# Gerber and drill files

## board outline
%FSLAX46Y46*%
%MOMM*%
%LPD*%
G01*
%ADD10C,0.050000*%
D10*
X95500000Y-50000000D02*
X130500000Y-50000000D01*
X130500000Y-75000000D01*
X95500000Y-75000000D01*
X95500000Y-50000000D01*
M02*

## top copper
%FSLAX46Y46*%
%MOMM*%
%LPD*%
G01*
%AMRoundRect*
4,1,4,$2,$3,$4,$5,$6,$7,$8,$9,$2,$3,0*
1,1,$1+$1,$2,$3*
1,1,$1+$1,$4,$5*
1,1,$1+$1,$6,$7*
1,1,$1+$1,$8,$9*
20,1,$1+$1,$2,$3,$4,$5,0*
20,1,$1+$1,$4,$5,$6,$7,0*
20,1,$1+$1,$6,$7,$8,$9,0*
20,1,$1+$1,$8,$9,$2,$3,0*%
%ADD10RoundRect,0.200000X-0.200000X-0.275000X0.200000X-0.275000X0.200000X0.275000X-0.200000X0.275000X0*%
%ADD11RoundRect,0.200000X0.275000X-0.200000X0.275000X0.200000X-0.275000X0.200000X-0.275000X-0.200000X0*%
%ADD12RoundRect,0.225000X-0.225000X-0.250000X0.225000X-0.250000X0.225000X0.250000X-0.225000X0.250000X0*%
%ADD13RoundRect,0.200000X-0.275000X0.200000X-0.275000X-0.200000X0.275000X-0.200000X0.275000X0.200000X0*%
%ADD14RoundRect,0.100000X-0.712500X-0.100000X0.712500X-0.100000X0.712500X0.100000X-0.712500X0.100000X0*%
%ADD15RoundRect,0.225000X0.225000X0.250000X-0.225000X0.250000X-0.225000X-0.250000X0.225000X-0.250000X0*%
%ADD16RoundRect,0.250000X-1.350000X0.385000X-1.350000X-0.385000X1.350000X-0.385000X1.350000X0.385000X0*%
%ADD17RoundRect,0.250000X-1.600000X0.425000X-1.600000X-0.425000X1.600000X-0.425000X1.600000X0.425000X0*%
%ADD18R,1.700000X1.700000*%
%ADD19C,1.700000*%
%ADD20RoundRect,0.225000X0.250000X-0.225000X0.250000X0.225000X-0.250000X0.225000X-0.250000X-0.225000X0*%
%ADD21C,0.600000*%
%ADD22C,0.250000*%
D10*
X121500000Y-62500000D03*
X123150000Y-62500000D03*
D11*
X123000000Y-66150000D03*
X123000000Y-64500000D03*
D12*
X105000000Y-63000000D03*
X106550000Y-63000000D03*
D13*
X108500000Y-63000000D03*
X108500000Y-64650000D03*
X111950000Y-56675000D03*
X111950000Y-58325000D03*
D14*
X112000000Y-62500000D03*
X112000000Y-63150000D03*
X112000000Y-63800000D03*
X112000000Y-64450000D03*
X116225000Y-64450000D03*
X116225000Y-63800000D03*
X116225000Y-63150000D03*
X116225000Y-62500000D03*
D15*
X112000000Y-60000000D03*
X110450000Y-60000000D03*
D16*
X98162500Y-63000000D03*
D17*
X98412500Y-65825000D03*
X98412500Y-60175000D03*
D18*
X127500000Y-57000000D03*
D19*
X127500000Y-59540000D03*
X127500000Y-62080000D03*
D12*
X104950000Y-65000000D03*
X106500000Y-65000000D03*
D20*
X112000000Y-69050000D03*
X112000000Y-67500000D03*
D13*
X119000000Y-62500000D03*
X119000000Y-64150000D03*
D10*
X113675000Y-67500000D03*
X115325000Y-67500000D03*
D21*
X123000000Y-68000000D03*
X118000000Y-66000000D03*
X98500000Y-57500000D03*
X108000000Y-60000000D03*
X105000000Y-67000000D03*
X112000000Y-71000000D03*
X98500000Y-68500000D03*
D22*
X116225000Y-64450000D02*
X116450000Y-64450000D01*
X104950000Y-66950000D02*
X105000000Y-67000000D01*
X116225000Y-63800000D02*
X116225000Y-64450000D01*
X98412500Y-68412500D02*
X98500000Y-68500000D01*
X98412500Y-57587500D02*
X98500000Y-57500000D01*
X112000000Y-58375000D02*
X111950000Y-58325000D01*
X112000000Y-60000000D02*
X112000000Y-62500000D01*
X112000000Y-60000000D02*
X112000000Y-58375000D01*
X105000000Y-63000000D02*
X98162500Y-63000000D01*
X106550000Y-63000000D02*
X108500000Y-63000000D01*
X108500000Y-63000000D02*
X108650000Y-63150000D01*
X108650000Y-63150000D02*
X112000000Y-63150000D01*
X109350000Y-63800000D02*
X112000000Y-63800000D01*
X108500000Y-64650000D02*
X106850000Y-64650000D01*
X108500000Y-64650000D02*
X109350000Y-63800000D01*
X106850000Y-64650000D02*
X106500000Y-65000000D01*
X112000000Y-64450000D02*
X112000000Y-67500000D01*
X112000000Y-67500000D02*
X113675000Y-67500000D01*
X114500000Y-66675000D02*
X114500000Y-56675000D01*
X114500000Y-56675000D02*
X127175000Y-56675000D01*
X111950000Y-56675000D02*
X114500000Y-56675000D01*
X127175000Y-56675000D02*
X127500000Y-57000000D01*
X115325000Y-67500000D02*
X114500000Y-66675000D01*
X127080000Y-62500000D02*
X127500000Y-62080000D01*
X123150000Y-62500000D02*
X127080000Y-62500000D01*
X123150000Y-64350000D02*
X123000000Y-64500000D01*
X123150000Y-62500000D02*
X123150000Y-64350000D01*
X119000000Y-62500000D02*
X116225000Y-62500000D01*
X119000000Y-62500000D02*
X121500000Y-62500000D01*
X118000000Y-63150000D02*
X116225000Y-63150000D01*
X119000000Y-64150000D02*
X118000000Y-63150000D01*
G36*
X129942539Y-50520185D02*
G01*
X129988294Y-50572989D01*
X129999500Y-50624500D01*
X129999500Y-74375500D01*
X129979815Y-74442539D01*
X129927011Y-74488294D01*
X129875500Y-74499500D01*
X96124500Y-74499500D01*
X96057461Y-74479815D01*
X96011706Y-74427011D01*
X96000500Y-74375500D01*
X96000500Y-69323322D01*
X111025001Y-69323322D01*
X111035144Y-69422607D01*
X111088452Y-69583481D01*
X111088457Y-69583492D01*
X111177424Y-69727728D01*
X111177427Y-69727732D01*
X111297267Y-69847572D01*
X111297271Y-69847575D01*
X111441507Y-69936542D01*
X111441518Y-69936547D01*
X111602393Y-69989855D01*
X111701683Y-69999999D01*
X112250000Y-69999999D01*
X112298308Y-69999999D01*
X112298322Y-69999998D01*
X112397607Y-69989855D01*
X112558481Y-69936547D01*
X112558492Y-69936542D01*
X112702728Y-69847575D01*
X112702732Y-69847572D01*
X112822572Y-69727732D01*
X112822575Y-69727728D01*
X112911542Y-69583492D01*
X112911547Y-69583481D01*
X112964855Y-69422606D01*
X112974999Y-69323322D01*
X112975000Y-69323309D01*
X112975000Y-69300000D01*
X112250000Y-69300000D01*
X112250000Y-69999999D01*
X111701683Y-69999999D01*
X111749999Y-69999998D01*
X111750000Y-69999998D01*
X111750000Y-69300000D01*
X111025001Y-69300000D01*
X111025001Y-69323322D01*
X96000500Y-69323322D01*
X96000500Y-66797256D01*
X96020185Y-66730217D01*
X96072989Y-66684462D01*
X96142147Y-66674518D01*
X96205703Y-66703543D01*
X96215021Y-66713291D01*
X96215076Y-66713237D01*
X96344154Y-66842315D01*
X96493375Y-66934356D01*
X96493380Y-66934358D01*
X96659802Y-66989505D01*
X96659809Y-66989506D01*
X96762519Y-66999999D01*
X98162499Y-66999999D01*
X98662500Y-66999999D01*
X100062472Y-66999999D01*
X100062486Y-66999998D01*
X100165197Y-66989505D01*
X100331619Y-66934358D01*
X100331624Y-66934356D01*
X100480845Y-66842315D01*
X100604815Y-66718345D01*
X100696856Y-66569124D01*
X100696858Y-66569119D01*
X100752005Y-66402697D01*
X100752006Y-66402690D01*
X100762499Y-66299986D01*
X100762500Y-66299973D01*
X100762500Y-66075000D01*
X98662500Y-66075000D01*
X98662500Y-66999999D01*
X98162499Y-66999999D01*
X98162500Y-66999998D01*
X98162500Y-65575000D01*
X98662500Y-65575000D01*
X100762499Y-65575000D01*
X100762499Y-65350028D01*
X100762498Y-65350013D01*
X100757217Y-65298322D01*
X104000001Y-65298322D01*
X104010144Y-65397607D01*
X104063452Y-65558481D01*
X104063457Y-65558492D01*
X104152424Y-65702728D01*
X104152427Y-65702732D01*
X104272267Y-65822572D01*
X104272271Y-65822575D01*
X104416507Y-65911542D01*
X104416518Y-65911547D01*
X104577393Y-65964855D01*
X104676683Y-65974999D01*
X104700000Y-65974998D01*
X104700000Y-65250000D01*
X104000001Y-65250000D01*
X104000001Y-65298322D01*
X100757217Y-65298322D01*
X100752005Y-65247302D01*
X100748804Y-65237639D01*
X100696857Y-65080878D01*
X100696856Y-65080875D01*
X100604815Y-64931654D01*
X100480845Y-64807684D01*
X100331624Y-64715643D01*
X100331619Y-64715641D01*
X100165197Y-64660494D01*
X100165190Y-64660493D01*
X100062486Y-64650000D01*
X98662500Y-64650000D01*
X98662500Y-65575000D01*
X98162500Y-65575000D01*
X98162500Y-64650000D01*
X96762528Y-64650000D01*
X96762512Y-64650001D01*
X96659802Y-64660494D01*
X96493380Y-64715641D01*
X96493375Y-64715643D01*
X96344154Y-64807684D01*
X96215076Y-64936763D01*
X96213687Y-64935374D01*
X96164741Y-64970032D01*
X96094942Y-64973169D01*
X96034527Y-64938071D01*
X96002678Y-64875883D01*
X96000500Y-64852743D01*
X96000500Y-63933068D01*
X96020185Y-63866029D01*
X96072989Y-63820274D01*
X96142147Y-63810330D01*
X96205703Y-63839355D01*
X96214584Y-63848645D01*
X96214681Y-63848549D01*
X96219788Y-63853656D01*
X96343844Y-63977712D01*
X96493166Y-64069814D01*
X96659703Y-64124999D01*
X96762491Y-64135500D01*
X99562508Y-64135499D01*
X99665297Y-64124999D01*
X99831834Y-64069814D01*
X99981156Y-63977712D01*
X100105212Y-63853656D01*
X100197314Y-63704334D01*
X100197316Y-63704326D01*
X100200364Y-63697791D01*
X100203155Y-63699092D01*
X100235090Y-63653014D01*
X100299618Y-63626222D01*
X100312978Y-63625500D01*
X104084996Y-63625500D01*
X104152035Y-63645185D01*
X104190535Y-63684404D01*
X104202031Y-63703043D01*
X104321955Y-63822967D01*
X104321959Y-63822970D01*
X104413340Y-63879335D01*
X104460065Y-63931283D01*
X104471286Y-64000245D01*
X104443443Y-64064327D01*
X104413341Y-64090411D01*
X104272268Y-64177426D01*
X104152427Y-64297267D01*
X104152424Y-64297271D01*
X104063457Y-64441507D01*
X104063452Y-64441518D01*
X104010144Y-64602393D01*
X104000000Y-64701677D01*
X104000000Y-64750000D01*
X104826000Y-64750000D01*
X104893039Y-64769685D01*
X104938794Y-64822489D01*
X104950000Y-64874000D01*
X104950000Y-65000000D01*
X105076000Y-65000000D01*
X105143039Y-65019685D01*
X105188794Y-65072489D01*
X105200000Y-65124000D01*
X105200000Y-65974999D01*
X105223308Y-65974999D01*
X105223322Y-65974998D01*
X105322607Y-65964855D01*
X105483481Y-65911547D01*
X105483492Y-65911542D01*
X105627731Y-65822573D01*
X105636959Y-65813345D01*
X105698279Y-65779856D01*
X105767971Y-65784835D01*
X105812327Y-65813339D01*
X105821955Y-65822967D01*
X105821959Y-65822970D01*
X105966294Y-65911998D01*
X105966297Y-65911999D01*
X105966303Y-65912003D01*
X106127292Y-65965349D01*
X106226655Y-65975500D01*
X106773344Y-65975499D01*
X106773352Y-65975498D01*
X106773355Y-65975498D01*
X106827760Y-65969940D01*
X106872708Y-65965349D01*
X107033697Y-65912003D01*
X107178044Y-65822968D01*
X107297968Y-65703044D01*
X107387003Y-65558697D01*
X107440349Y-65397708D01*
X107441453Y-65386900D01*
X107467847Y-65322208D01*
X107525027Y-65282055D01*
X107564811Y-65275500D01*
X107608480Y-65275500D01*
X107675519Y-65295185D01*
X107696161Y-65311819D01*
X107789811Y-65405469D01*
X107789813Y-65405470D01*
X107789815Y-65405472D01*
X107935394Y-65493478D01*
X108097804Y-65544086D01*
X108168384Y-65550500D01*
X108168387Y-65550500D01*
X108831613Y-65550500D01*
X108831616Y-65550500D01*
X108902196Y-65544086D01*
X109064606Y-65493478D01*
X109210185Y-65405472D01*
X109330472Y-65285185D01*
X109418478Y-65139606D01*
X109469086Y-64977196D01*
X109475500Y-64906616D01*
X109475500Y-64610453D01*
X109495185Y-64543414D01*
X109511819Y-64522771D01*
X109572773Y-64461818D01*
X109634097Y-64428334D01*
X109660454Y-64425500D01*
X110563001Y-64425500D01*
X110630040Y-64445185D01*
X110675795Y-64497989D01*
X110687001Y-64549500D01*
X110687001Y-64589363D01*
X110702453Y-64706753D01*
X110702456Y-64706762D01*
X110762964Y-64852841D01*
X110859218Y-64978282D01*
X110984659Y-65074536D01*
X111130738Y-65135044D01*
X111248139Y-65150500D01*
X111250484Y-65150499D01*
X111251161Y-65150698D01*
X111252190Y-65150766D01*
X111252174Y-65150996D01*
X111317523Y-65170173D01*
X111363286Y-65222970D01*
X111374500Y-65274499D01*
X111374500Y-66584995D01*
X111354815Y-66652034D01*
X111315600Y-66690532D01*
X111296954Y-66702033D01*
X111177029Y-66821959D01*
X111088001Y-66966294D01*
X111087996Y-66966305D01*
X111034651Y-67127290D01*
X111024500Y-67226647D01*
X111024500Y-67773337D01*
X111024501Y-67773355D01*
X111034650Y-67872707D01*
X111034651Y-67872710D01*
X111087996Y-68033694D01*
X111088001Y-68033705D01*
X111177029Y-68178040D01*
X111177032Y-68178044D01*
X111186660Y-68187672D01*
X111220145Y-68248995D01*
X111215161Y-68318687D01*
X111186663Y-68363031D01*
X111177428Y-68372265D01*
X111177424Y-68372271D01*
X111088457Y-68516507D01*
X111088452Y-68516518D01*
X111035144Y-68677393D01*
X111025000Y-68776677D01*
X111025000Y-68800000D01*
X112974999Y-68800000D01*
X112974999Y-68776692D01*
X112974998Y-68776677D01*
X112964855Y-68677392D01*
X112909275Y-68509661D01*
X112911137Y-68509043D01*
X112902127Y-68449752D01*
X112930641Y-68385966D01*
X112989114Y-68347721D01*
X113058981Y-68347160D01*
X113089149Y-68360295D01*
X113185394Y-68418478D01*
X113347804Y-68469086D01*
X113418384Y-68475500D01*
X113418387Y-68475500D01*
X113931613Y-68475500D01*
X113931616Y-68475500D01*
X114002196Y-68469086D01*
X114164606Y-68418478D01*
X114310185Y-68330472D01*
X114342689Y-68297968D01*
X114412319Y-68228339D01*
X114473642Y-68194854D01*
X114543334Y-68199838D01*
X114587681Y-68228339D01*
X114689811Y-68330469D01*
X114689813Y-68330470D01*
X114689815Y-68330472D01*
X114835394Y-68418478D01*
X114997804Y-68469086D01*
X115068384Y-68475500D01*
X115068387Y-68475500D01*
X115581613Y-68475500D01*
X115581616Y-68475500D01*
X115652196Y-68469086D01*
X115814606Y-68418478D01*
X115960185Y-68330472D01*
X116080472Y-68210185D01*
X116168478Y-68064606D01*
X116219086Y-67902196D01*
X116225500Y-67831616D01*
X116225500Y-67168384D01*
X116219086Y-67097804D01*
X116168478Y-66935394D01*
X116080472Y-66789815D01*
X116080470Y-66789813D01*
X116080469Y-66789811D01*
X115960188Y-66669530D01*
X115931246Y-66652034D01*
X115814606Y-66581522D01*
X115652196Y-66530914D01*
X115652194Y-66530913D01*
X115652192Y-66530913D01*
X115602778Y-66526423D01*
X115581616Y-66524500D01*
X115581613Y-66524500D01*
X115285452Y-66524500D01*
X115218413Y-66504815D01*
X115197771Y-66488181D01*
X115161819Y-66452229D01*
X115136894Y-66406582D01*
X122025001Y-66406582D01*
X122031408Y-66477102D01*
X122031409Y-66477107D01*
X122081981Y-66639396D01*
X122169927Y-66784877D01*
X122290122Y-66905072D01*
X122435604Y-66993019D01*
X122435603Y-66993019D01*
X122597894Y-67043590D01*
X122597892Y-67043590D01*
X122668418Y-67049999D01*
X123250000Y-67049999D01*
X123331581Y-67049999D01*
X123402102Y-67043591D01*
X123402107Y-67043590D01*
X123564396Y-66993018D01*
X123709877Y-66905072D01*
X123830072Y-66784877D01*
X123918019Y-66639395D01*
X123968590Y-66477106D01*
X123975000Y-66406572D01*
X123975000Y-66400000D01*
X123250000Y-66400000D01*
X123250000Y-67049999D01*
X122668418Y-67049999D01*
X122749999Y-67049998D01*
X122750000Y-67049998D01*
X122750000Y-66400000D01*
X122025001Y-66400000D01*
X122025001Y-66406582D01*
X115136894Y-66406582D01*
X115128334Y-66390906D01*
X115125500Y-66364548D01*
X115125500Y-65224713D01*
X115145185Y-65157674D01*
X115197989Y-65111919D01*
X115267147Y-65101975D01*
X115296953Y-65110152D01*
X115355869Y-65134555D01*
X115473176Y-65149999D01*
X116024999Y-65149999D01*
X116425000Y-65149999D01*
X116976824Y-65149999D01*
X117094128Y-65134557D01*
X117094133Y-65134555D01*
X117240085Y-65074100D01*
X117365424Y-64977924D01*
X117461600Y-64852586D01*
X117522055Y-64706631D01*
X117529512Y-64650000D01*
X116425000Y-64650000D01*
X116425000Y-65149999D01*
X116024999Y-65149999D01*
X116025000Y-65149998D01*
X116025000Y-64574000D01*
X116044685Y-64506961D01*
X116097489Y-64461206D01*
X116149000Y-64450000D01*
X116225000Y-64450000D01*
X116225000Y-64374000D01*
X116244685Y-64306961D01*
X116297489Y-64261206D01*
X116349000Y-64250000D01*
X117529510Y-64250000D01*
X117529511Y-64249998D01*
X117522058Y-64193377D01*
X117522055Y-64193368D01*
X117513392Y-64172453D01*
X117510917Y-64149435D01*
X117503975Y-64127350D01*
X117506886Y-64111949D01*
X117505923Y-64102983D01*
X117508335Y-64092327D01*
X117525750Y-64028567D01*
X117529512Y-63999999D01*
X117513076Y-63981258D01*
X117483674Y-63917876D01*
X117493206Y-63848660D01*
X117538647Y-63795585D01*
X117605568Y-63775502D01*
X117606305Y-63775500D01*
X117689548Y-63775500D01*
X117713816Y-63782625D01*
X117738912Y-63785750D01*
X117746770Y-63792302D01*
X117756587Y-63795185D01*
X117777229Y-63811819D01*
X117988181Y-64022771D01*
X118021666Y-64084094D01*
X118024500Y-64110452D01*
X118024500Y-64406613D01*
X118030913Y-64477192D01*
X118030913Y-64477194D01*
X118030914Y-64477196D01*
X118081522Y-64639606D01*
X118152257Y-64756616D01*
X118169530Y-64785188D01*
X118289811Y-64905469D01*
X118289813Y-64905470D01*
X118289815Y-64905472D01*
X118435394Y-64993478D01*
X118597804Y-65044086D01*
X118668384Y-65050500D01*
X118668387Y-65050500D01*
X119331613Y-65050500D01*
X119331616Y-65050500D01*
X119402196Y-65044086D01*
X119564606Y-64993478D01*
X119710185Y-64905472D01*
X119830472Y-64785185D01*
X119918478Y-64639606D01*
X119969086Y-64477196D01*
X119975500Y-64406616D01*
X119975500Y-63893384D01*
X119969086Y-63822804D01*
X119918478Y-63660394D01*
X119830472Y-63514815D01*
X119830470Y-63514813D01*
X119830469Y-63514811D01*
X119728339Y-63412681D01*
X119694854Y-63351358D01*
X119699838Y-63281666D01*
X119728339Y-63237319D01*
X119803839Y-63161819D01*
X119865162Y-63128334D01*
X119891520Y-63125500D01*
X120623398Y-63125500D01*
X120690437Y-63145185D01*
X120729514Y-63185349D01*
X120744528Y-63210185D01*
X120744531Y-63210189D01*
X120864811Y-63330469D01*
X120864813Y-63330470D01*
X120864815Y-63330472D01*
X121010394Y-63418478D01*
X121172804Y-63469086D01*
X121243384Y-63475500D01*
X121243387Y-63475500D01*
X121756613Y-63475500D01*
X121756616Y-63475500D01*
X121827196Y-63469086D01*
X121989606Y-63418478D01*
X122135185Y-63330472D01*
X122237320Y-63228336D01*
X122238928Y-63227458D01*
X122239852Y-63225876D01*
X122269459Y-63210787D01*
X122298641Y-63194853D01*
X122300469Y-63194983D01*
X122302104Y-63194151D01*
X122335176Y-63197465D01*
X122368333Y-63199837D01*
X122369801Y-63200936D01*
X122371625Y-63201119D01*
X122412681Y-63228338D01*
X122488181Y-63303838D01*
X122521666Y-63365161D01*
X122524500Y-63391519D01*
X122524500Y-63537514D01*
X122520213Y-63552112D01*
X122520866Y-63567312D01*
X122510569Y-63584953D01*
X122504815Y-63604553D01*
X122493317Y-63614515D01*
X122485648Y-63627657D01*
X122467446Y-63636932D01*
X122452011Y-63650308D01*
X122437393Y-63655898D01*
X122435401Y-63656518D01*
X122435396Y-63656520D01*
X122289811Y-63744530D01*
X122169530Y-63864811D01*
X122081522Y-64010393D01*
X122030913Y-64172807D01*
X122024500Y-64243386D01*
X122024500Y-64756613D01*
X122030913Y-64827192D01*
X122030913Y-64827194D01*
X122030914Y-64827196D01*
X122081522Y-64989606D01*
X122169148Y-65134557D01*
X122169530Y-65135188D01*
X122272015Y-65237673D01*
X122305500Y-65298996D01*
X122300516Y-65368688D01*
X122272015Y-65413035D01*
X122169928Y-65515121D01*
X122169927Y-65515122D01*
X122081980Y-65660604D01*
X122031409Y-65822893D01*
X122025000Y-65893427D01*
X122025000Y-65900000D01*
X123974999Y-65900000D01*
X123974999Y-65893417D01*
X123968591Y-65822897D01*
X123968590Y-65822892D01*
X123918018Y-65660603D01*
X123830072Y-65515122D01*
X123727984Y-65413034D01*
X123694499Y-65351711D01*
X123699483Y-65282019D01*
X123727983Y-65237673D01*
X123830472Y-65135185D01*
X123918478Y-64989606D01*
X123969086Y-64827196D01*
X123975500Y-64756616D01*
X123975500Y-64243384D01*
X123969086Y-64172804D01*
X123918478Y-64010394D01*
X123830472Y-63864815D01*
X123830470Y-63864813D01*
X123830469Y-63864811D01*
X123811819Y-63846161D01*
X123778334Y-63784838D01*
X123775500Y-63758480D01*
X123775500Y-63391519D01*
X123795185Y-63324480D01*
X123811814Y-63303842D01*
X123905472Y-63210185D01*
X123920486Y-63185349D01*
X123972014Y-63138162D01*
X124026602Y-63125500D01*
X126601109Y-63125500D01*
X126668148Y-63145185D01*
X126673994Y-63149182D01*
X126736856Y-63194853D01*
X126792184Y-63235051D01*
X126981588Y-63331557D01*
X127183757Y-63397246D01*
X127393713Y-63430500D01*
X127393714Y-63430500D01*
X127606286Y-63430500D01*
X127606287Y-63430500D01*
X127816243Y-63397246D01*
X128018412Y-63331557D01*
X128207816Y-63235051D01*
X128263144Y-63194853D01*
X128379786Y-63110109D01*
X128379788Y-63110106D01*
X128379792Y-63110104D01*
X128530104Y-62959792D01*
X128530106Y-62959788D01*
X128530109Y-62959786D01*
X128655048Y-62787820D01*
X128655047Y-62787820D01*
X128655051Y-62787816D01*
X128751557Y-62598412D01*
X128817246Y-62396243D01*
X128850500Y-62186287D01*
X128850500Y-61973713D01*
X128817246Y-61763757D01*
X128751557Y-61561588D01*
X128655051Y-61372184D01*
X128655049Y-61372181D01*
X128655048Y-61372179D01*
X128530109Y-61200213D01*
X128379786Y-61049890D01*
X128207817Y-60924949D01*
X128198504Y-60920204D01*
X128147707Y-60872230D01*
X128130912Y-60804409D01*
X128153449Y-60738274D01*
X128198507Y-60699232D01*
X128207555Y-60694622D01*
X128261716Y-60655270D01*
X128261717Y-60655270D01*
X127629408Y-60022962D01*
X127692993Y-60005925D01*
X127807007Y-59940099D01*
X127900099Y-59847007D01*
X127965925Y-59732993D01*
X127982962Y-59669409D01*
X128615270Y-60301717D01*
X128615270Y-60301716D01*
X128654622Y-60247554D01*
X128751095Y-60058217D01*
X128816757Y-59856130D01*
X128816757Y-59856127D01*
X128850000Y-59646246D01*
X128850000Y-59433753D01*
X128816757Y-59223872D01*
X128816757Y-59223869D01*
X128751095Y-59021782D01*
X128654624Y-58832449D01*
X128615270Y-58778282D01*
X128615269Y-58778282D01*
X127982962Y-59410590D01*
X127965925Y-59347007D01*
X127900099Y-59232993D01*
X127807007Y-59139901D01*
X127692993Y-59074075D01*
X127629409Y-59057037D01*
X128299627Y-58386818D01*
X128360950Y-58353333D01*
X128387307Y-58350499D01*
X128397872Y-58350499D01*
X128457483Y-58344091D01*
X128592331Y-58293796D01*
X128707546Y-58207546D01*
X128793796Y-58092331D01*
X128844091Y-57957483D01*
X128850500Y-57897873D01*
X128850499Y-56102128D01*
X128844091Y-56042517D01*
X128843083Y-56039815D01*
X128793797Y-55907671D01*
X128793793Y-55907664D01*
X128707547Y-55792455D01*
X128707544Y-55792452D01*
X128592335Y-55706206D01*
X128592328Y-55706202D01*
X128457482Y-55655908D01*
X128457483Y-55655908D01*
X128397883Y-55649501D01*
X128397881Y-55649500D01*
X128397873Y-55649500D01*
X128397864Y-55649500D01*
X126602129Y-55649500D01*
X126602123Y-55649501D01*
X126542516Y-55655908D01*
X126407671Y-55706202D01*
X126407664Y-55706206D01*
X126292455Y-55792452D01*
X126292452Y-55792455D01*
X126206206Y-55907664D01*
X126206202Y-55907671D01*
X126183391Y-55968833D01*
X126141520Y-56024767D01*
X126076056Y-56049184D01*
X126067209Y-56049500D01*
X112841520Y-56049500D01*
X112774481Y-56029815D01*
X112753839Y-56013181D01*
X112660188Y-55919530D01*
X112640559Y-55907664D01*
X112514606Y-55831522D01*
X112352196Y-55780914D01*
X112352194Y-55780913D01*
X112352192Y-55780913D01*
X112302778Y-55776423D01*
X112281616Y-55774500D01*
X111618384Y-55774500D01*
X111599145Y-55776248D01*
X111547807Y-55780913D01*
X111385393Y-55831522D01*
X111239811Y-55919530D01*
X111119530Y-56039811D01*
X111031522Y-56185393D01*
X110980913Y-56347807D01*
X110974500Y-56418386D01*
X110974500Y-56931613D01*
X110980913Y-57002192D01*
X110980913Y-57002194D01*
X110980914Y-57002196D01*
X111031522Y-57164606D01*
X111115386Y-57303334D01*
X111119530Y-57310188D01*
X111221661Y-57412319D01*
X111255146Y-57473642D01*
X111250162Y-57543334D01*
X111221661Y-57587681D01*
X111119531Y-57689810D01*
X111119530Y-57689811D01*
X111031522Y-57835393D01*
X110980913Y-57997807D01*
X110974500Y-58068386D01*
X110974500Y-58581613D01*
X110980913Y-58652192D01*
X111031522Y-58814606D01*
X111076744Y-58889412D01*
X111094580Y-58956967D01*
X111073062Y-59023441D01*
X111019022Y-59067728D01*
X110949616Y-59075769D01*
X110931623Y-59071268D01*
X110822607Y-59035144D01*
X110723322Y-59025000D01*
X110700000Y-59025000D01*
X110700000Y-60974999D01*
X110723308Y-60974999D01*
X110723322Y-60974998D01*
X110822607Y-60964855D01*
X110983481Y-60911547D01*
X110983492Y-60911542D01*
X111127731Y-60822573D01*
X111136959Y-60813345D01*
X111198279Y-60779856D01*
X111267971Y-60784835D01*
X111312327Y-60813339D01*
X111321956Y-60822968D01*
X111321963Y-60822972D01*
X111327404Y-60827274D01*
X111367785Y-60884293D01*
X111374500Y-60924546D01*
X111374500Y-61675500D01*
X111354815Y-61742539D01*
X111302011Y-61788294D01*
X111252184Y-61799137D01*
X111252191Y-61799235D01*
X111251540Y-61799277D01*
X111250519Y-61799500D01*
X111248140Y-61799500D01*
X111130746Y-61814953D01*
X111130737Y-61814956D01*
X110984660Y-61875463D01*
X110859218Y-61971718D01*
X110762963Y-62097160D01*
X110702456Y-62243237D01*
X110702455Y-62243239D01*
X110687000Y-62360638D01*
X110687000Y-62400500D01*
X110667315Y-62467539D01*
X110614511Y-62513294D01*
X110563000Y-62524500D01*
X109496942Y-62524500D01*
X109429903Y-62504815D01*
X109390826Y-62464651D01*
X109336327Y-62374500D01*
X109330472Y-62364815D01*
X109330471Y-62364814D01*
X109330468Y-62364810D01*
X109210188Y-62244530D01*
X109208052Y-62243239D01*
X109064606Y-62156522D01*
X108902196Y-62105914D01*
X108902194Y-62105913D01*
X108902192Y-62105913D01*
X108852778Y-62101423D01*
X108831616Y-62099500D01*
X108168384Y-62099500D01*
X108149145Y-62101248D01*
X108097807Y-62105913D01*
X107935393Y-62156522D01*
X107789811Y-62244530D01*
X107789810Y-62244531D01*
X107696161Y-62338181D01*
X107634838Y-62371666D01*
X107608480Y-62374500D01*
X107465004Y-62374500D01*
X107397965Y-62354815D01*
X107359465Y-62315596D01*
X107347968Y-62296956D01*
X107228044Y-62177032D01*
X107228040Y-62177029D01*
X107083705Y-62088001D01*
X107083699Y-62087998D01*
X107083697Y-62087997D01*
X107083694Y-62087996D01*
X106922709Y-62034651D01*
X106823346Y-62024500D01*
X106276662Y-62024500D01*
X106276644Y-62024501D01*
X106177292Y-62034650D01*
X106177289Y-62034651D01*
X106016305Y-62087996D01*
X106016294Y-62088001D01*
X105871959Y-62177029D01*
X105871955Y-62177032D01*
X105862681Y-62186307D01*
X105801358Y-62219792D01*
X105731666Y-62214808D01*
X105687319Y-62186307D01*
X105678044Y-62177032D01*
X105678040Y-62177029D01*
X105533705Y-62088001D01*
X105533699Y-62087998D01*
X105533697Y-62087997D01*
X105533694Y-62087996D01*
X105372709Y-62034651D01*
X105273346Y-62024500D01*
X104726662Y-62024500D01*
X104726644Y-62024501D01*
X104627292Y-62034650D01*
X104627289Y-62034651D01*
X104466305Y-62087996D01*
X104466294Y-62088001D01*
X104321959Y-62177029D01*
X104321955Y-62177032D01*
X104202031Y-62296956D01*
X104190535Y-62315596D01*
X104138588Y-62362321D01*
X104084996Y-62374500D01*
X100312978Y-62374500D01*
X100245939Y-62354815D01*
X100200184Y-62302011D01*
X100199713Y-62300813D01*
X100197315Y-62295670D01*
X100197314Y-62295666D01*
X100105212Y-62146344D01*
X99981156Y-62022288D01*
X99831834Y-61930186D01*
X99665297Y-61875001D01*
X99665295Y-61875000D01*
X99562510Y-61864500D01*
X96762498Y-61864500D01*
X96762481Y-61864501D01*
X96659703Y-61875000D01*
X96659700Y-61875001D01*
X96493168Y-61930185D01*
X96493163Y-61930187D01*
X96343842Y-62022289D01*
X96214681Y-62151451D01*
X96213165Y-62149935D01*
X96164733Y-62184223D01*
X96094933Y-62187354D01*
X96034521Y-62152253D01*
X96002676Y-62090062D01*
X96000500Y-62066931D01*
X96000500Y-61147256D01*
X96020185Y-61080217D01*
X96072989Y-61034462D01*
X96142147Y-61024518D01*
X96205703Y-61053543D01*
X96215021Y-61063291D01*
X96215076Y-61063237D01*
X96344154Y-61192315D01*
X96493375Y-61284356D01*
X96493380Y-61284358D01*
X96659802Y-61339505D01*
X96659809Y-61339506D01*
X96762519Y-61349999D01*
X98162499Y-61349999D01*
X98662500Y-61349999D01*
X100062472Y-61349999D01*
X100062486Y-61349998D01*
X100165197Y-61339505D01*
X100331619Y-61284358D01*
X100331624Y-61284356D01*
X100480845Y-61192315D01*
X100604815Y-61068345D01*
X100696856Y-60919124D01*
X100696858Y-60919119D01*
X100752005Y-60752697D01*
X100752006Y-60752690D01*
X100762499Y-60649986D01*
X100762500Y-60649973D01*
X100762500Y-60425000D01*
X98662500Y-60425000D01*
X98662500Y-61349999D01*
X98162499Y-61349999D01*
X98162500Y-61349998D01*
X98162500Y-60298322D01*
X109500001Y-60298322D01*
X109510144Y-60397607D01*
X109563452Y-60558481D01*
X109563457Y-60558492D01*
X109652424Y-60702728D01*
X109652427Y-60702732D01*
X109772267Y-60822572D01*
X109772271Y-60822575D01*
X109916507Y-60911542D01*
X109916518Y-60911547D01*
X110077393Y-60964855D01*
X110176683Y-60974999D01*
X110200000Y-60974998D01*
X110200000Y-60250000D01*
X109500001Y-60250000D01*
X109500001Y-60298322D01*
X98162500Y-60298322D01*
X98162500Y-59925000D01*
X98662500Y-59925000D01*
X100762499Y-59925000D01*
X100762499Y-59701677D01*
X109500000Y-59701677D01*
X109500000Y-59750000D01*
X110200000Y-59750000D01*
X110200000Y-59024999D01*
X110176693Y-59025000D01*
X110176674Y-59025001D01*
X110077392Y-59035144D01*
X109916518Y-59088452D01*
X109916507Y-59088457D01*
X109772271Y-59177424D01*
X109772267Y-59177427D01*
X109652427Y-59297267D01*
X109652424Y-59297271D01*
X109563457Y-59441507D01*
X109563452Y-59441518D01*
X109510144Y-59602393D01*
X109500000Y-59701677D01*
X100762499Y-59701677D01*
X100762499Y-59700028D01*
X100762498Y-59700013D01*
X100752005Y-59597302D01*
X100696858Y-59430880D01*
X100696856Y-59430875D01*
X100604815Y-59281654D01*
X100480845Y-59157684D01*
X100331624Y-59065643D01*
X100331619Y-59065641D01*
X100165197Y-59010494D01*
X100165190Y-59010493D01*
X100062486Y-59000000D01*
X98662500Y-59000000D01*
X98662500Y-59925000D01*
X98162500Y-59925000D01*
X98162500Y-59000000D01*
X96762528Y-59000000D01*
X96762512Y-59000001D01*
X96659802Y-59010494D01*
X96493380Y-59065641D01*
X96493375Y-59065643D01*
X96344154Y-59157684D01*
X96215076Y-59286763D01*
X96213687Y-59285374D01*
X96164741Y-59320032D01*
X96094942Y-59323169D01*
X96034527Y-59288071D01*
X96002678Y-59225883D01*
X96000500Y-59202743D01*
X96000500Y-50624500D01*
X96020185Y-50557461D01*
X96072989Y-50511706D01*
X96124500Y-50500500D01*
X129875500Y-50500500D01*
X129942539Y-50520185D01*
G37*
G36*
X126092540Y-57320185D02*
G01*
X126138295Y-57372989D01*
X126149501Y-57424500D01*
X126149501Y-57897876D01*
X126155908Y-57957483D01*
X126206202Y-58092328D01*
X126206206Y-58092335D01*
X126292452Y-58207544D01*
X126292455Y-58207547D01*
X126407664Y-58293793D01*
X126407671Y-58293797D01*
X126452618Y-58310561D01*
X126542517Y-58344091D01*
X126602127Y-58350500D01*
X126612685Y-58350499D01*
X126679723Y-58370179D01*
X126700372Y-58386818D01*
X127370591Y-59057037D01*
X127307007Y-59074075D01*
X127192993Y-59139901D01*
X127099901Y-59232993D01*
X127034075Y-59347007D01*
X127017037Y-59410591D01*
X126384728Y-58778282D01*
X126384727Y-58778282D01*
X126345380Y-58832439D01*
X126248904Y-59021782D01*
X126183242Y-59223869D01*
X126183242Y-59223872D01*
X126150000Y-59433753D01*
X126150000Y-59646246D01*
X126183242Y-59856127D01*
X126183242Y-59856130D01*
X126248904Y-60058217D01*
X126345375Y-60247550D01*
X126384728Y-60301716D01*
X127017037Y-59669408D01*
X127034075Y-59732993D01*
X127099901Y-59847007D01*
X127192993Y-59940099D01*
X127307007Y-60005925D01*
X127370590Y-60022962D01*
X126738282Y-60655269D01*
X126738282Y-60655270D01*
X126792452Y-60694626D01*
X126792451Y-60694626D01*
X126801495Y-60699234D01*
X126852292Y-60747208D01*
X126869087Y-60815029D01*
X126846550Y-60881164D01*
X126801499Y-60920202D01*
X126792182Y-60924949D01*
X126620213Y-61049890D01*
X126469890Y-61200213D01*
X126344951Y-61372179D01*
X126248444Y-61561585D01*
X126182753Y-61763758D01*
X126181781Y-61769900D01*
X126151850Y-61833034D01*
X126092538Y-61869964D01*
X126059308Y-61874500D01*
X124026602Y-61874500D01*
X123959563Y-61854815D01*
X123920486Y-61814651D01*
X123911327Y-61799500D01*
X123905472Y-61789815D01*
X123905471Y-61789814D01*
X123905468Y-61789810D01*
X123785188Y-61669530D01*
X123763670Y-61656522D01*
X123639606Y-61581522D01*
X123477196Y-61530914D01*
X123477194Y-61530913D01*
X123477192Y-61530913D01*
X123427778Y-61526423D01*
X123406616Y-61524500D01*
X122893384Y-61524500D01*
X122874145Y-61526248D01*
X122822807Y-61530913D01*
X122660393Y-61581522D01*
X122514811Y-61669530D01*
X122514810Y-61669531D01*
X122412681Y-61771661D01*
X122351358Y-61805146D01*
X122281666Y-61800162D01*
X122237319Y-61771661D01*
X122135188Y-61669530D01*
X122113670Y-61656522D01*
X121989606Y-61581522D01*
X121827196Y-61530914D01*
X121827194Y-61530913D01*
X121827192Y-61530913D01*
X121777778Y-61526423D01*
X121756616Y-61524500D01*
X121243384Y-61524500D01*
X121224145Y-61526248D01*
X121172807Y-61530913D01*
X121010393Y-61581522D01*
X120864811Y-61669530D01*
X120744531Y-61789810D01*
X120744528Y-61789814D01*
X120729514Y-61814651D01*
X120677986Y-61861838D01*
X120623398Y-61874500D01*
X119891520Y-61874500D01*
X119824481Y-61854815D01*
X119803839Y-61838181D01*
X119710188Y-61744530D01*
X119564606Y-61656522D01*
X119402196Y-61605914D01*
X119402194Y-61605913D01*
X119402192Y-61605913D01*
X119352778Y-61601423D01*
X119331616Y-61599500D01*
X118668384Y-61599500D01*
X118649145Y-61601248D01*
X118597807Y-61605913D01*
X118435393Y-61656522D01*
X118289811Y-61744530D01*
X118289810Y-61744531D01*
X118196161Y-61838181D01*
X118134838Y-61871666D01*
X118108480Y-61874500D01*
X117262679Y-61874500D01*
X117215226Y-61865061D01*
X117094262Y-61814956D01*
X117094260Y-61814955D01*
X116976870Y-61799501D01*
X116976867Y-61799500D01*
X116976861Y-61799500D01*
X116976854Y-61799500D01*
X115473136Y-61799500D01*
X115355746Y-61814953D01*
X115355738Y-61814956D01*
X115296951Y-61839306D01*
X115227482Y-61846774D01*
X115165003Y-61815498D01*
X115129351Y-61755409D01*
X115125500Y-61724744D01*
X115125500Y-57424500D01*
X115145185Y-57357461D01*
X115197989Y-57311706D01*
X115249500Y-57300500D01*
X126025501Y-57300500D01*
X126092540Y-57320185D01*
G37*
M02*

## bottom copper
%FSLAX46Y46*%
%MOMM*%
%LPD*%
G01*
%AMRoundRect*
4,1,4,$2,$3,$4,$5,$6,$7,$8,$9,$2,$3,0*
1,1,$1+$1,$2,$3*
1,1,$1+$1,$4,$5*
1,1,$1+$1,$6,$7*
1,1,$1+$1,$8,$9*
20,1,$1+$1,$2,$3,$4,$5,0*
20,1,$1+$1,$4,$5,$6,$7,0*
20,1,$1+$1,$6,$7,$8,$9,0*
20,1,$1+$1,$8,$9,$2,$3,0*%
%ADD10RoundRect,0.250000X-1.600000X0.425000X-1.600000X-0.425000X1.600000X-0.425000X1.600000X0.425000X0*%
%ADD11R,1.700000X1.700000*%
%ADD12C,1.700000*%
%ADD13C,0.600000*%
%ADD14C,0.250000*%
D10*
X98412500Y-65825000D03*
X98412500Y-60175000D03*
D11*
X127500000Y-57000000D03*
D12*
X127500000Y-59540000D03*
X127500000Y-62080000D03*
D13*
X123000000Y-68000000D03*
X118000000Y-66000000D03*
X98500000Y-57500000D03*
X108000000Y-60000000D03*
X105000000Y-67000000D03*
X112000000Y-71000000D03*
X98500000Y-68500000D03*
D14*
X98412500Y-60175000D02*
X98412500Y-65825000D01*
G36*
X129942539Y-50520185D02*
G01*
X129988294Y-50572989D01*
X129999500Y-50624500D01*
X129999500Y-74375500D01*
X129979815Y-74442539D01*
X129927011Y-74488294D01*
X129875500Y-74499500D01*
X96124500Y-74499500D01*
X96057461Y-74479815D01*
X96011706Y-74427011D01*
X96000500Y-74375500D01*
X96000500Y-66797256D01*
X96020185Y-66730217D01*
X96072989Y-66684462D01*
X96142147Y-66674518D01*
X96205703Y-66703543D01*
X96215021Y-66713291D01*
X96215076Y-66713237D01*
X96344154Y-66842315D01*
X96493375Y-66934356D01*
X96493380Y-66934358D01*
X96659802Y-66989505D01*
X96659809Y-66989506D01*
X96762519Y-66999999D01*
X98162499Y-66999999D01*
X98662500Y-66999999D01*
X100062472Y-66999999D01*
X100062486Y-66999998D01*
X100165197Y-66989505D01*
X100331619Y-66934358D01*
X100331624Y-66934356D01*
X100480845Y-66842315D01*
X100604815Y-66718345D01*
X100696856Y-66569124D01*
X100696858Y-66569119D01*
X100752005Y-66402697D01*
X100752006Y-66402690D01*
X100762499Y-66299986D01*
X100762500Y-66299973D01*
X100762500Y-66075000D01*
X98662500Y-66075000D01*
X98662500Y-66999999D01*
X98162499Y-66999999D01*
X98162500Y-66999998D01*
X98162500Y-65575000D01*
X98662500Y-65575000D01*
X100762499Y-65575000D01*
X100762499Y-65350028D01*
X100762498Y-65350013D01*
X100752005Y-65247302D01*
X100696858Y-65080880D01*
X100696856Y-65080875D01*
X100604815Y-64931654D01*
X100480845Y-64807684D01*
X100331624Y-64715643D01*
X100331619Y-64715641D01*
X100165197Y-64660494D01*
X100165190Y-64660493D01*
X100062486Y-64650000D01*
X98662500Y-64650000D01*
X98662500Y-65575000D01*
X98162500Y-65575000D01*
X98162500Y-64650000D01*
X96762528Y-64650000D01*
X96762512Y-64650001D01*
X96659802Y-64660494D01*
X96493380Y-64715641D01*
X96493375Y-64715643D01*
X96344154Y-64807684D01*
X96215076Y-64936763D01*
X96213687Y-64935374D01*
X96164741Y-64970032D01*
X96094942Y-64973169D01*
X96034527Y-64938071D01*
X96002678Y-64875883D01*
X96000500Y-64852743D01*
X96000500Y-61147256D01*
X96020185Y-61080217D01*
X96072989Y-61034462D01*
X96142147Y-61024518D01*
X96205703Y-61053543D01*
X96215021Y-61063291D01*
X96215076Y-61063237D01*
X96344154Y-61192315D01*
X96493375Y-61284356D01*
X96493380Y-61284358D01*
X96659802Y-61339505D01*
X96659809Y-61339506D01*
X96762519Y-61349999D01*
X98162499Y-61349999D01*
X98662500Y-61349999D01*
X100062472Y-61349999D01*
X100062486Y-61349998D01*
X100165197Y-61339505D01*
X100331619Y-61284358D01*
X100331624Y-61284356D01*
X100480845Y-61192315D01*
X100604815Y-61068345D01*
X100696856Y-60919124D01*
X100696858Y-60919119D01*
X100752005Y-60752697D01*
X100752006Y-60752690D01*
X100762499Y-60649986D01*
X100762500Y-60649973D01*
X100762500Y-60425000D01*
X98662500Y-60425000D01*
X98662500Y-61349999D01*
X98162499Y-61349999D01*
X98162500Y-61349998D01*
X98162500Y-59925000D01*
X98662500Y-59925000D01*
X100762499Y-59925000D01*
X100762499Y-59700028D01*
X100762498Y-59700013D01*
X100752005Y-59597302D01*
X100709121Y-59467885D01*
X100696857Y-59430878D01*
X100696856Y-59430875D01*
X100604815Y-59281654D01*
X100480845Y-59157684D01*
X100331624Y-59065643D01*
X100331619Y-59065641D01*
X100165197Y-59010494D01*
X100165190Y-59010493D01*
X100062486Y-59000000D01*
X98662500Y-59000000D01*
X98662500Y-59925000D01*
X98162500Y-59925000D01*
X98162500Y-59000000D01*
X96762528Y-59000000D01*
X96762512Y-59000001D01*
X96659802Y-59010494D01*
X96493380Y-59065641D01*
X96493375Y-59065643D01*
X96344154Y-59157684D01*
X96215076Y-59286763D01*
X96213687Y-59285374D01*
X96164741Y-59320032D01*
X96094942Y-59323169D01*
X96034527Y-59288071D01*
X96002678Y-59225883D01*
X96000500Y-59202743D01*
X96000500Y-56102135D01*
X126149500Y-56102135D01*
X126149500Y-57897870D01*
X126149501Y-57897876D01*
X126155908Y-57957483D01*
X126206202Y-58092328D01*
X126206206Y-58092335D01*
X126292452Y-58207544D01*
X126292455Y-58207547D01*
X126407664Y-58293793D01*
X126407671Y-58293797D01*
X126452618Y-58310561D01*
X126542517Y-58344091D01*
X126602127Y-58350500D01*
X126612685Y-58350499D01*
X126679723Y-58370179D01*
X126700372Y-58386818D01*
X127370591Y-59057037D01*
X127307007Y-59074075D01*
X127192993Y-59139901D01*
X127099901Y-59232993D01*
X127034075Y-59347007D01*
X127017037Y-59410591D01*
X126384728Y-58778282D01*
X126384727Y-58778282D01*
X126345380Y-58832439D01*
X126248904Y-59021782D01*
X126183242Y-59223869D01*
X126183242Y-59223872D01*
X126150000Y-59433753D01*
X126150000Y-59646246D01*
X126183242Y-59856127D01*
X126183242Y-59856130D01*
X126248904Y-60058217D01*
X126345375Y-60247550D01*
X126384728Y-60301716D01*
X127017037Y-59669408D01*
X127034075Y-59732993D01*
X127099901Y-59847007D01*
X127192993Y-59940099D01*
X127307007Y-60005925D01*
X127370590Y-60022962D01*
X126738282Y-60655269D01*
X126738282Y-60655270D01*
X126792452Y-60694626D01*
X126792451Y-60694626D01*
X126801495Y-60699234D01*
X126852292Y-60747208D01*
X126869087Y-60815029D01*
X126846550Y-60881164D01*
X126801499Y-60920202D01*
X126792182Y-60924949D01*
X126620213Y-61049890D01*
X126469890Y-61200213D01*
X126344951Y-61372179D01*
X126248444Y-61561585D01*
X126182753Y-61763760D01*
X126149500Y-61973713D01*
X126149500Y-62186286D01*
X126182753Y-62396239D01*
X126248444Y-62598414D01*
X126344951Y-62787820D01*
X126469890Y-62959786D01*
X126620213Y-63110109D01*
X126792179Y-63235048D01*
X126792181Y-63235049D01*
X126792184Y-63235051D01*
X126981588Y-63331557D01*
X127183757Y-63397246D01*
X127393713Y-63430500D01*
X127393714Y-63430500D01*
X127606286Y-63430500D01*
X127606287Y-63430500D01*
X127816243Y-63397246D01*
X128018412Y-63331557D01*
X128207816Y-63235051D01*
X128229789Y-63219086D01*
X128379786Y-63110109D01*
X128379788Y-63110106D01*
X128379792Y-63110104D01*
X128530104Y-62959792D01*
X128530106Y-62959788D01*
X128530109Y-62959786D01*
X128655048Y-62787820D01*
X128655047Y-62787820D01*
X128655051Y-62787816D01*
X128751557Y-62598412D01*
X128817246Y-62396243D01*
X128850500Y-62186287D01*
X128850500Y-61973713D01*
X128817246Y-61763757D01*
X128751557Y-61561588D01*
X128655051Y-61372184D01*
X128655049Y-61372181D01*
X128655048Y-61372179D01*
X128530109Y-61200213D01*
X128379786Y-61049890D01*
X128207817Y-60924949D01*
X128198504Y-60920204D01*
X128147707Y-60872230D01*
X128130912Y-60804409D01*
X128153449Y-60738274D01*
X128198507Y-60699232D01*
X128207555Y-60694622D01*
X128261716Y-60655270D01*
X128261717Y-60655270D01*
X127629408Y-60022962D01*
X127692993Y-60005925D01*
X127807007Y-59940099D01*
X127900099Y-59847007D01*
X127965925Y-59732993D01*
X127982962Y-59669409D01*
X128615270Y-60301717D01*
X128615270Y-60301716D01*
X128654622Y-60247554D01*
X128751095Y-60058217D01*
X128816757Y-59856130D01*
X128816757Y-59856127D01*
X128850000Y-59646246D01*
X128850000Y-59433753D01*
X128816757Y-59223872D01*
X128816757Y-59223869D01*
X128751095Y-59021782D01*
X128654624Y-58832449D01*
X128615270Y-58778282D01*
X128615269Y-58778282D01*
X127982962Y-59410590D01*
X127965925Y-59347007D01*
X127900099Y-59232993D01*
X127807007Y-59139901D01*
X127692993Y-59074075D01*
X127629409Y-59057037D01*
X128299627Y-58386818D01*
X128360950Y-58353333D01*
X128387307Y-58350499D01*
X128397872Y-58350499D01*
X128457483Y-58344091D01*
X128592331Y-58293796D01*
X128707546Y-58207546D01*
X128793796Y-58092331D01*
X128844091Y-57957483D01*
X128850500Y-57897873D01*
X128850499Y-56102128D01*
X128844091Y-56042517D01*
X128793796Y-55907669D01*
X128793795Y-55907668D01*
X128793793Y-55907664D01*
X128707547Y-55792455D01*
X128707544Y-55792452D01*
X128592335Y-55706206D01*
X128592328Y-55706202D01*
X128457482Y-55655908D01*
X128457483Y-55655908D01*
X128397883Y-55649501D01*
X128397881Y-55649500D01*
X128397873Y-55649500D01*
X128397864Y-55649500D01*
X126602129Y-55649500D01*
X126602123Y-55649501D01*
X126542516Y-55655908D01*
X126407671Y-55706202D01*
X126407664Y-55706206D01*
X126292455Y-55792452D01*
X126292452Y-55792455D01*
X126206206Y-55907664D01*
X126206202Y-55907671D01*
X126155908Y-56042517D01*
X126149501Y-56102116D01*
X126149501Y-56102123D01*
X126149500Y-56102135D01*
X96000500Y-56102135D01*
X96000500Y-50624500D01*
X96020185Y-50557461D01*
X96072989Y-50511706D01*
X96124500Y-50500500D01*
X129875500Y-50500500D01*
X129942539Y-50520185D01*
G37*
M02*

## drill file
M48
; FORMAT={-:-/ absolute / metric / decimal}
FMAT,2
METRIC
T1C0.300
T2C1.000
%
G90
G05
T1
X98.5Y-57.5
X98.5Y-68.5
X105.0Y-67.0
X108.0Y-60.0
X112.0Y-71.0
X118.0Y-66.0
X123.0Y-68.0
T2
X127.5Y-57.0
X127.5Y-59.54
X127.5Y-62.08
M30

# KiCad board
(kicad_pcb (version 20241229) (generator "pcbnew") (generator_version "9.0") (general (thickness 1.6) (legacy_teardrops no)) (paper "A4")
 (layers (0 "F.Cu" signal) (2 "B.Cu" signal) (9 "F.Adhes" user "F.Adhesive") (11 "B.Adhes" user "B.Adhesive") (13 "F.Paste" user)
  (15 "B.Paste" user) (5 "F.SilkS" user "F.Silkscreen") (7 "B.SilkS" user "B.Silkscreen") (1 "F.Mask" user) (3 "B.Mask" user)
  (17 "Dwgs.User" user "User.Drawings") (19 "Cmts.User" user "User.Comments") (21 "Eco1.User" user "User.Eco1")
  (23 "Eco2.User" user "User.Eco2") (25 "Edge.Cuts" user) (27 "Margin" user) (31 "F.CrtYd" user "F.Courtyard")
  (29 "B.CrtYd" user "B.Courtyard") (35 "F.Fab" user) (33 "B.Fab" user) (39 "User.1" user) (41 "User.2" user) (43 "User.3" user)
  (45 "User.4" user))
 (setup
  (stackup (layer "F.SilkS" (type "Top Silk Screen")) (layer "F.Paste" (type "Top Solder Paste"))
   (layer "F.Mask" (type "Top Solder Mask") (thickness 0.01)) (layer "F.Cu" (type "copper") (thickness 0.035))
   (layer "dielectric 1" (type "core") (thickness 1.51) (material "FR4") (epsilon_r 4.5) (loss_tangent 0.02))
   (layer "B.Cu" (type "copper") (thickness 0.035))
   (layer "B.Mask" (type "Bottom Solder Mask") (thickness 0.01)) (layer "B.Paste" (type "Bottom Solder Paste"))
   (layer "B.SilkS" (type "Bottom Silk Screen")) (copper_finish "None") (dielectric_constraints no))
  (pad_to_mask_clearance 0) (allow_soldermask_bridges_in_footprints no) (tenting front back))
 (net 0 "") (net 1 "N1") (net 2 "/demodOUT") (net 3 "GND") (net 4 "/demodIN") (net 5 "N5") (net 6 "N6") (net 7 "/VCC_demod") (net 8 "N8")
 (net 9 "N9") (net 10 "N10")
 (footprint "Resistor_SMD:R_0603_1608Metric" (layer "F.Cu") (at 122.325 62.5)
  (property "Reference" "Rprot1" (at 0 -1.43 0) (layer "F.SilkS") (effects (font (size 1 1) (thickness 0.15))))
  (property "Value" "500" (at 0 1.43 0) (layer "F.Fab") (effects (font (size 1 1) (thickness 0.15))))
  (pad "1" smd roundrect (at -0.825 0) (size 0.8 0.95) (layers "F.Cu" "F.Mask" "F.Paste") (roundrect_rratio 0.25) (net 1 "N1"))
  (pad "2" smd roundrect (at 0.825 0) (size 0.8 0.95) (layers "F.Cu" "F.Mask" "F.Paste") (roundrect_rratio 0.25) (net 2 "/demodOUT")))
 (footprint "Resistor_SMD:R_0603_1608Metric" (layer "F.Cu") (at 123 65.325 90)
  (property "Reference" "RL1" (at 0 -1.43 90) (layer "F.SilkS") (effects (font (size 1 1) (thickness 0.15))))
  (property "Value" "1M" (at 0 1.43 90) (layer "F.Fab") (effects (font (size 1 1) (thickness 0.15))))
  (pad "1" smd roundrect (at -0.825 0 90) (size 0.8 0.95) (layers "F.Cu" "F.Mask" "F.Paste") (roundrect_rratio 0.25) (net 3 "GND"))
  (pad "2" smd roundrect (at 0.825 0 90) (size 0.8 0.95) (layers "F.Cu" "F.Mask" "F.Paste") (roundrect_rratio 0.25) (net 2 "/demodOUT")))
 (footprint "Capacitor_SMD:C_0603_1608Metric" (layer "F.Cu") (at 105.775 63)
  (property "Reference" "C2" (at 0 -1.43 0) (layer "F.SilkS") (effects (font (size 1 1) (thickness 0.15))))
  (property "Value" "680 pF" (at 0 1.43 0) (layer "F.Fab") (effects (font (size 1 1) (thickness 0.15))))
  (pad "1" smd roundrect (at -0.775 0) (size 0.9 0.95) (layers "F.Cu" "F.Mask" "F.Paste") (roundrect_rratio 0.25) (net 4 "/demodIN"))
  (pad "2" smd roundrect (at 0.775 0) (size 0.9 0.95) (layers "F.Cu" "F.Mask" "F.Paste") (roundrect_rratio 0.25) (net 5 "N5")))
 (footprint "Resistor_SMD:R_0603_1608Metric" (layer "F.Cu") (at 108.5 63.825 -90)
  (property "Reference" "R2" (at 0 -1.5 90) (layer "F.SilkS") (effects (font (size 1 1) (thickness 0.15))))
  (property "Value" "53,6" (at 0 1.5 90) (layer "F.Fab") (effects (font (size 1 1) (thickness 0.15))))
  (pad "1" smd roundrect (at -0.825 0 270) (size 0.8 0.95) (layers "F.Cu" "F.Mask" "F.Paste") (roundrect_rratio 0.25) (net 5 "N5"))
  (pad "2" smd roundrect (at 0.825 0 270) (size 0.8 0.95) (layers "F.Cu" "F.Mask" "F.Paste") (roundrect_rratio 0.25) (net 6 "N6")))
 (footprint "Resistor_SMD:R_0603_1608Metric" (layer "F.Cu") (at 111.95 57.5 -90)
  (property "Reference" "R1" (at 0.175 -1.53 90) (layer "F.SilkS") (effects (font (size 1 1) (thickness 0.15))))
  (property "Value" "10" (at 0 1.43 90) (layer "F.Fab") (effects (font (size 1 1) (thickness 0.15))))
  (pad "1" smd roundrect (at -0.825 0 270) (size 0.8 0.95) (layers "F.Cu" "F.Mask" "F.Paste") (roundrect_rratio 0.25) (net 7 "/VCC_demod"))
  (pad "2" smd roundrect (at 0.825 0 270) (size 0.8 0.95) (layers "F.Cu" "F.Mask" "F.Paste") (roundrect_rratio 0.25) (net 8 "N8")))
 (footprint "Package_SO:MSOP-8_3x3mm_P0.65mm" (layer "F.Cu") (at 114.1125 63.475)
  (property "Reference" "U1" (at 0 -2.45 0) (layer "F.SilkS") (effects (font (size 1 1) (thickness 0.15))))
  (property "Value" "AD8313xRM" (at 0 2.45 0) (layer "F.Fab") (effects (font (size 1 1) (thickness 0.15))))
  (pad "1" smd roundrect (at -2.1125 -0.975) (size 1.625 0.4) (layers "F.Cu" "F.Mask" "F.Paste") (roundrect_rratio 0.25) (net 8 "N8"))
  (pad "2" smd roundrect (at -2.1125 -0.325) (size 1.625 0.4) (layers "F.Cu" "F.Mask" "F.Paste") (roundrect_rratio 0.25) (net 5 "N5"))
  (pad "3" smd roundrect (at -2.1125 0.325) (size 1.625 0.4) (layers "F.Cu" "F.Mask" "F.Paste") (roundrect_rratio 0.25) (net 6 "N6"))
  (pad "4" smd roundrect (at -2.1125 0.975) (size 1.625 0.4) (layers "F.Cu" "F.Mask" "F.Paste") (roundrect_rratio 0.25) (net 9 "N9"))
  (pad "5" smd roundrect (at 2.1125 0.975) (size 1.625 0.4) (layers "F.Cu" "F.Mask" "F.Paste") (roundrect_rratio 0.25) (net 3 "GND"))
  (pad "6" smd roundrect (at 2.1125 0.325) (size 1.625 0.4) (layers "F.Cu" "F.Mask" "F.Paste") (roundrect_rratio 0.25) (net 3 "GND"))
  (pad "7" smd roundrect (at 2.1125 -0.325) (size 1.625 0.4) (layers "F.Cu" "F.Mask" "F.Paste") (roundrect_rratio 0.25) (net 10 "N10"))
  (pad "8" smd roundrect (at 2.1125 -0.975) (size 1.625 0.4) (layers "F.Cu" "F.Mask" "F.Paste") (roundrect_rratio 0.25) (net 1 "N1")))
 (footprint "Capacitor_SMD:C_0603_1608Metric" (layer "F.Cu") (at 111.225 60 180)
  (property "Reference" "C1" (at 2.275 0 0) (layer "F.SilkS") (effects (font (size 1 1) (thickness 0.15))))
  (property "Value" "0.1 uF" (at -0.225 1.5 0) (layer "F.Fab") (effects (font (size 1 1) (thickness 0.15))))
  (pad "1" smd roundrect (at -0.775 0 180) (size 0.9 0.95) (layers "F.Cu" "F.Mask" "F.Paste") (roundrect_rratio 0.25) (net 8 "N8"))
  (pad "2" smd roundrect (at 0.775 0 180) (size 0.9 0.95) (layers "F.Cu" "F.Mask" "F.Paste") (roundrect_rratio 0.25) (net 3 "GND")))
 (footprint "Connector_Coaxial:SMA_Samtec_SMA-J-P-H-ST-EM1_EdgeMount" (layer "F.Cu") (at 98.1625 63 180)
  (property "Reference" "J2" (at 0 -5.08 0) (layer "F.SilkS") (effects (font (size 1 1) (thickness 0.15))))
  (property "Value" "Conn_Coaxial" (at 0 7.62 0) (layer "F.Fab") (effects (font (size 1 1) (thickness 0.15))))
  (pad "1" smd roundrect (at 0 0 270) (size 1.27 3.2) (layers "F.Cu" "F.Mask") (roundrect_rratio 0.1968503937) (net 4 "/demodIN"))
  (pad "2" smd roundrect (at -0.25 -2.825 270) (size 1.35 3.7) (layers "F.Cu" "F.Mask") (roundrect_rratio 0.1851851852) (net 3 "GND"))
  (pad "2" smd roundrect (at -0.25 -2.825 270) (size 1.35 3.7) (layers "B.Cu" "B.Mask") (roundrect_rratio 0.1851851852) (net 3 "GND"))
  (pad "2" smd roundrect (at -0.25 2.825 270) (size 1.35 3.7) (layers "F.Cu" "F.Mask") (roundrect_rratio 0.1851851852) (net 3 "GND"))
  (pad "2" smd roundrect (at -0.25 2.825 270) (size 1.35 3.7) (layers "B.Cu" "B.Mask") (roundrect_rratio 0.1851851852) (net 3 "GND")))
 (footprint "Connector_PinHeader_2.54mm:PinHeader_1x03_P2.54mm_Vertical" (layer "F.Cu") (at 127.5 57)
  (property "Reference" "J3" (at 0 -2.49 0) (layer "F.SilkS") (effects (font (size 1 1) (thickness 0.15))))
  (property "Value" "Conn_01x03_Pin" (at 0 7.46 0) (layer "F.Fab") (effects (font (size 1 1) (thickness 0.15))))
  (pad "1" thru_hole rect (at 0 0) (size 1.7 1.7) (drill 1) (layers "*.Cu" "*.Mask") (remove_unused_layers no) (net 7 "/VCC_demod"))
  (pad "2" thru_hole circle (at 0 2.54) (size 1.7 1.7) (drill 1) (layers "*.Cu" "*.Mask") (remove_unused_layers no) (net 3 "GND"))
  (pad "3" thru_hole circle (at 0 5.08) (size 1.7 1.7) (drill 1) (layers "*.Cu" "*.Mask") (remove_unused_layers no) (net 2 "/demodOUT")))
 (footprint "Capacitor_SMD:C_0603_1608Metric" (layer "F.Cu") (at 105.725 65)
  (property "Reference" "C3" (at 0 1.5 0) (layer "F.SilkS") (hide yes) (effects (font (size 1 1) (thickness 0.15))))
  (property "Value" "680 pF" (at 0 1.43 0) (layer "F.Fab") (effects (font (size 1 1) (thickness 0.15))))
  (pad "1" smd roundrect (at -0.775 0) (size 0.9 0.95) (layers "F.Cu" "F.Mask" "F.Paste") (roundrect_rratio 0.25) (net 3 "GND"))
  (pad "2" smd roundrect (at 0.775 0) (size 0.9 0.95) (layers "F.Cu" "F.Mask" "F.Paste") (roundrect_rratio 0.25) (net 6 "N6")))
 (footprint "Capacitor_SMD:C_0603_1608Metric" (layer "F.Cu") (at 112 68.275 90)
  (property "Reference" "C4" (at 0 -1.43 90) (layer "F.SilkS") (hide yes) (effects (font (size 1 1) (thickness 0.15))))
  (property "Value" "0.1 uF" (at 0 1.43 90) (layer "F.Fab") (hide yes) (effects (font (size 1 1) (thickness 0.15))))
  (pad "1" smd roundrect (at -0.775 0 90) (size 0.9 0.95) (layers "F.Cu" "F.Mask" "F.Paste") (roundrect_rratio 0.25) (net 3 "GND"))
  (pad "2" smd roundrect (at 0.775 0 90) (size 0.9 0.95) (layers "F.Cu" "F.Mask" "F.Paste") (roundrect_rratio 0.25) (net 9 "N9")))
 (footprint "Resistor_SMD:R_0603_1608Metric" (layer "F.Cu") (at 119 63.325 -90)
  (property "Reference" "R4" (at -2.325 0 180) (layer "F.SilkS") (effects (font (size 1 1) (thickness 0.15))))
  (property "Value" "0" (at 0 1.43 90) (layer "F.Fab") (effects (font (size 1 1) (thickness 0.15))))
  (pad "1" smd roundrect (at -0.825 0 270) (size 0.8 0.95) (layers "F.Cu" "F.Mask" "F.Paste") (roundrect_rratio 0.25) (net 1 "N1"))
  (pad "2" smd roundrect (at 0.825 0 270) (size 0.8 0.95) (layers "F.Cu" "F.Mask" "F.Paste") (roundrect_rratio 0.25) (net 10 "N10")))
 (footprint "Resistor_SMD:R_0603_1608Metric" (layer "F.Cu") (at 114.5 67.5)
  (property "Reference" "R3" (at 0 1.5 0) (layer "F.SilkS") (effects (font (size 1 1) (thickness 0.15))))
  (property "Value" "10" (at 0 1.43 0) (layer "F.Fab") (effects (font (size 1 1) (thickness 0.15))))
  (pad "1" smd roundrect (at -0.825 0) (size 0.8 0.95) (layers "F.Cu" "F.Mask" "F.Paste") (roundrect_rratio 0.25) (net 9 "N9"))
  (pad "2" smd roundrect (at 0.825 0) (size 0.8 0.95) (layers "F.Cu" "F.Mask" "F.Paste") (roundrect_rratio 0.25) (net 7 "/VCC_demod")))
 (gr_rect (start 95.5 50) (end 130.5 75) (stroke (width 0.05) (type solid)) (fill no) (layer "Edge.Cuts"))
 (segment (start 116.225 64.45) (end 116.45 64.45) (width 0.25) (layer "F.Cu") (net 3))
 (segment (start 104.95 66.95) (end 105 67) (width 0.25) (layer "F.Cu") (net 3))
 (segment (start 116.225 63.8) (end 116.225 64.45) (width 0.25) (layer "F.Cu") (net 3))
 (segment (start 98.4125 68.4125) (end 98.5 68.5) (width 0.25) (layer "F.Cu") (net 3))
 (segment (start 98.4125 57.5875) (end 98.5 57.5) (width 0.25) (layer "F.Cu") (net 3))
 (via (at 123 68) (size 0.6) (drill 0.3) (layers "F.Cu" "B.Cu") (free yes) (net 3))
 (via (at 118 66) (size 0.6) (drill 0.3) (layers "F.Cu" "B.Cu") (free yes) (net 3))
 (via (at 98.5 57.5) (size 0.6) (drill 0.3) (layers "F.Cu" "B.Cu") (free yes) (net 3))
 (via (at 108 60) (size 0.6) (drill 0.3) (layers "F.Cu" "B.Cu") (free yes) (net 3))
 (via (at 105 67) (size 0.6) (drill 0.3) (layers "F.Cu" "B.Cu") (free yes) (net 3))
 (via (at 112 71) (size 0.6) (drill 0.3) (layers "F.Cu" "B.Cu") (free yes) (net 3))
 (via (at 98.5 68.5) (size 0.6) (drill 0.3) (layers "F.Cu" "B.Cu") (free yes) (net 3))
 (segment (start 98.4125 60.175) (end 98.4125 65.825) (width 0.25) (layer "B.Cu") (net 3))
 (segment (start 112 58.375) (end 111.95 58.325) (width 0.25) (layer "F.Cu") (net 8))
 (segment (start 112 60) (end 112 62.5) (width 0.25) (layer "F.Cu") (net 8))
 (segment (start 112 60) (end 112 58.375) (width 0.25) (layer "F.Cu") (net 8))
 (segment (start 105 63) (end 98.1625 63) (width 0.25) (layer "F.Cu") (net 4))
 (segment (start 106.55 63) (end 108.5 63) (width 0.25) (layer "F.Cu") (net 5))
 (segment (start 108.5 63) (end 108.65 63.15) (width 0.25) (layer "F.Cu") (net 5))
 (segment (start 108.65 63.15) (end 112 63.15) (width 0.25) (layer "F.Cu") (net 5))
 (segment (start 109.35 63.8) (end 112 63.8) (width 0.25) (layer "F.Cu") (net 6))
 (segment (start 108.5 64.65) (end 106.85 64.65) (width 0.25) (layer "F.Cu") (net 6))
 (segment (start 108.5 64.65) (end 109.35 63.8) (width 0.25) (layer "F.Cu") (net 6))
 (segment (start 106.85 64.65) (end 106.5 65) (width 0.25) (layer "F.Cu") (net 6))
 (segment (start 112 64.45) (end 112 67.5) (width 0.25) (layer "F.Cu") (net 9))
 (segment (start 112 67.5) (end 113.675 67.5) (width 0.25) (layer "F.Cu") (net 9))
 (segment (start 114.5 66.675) (end 114.5 56.675) (width 0.25) (layer "F.Cu") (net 7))
 (segment (start 114.5 56.675) (end 127.175 56.675) (width 0.25) (layer "F.Cu") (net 7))
 (segment (start 111.95 56.675) (end 114.5 56.675) (width 0.25) (layer "F.Cu") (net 7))
 (segment (start 127.175 56.675) (end 127.5 57) (width 0.25) (layer "F.Cu") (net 7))
 (segment (start 115.325 67.5) (end 114.5 66.675) (width 0.25) (layer "F.Cu") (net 7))
 (segment (start 127.08 62.5) (end 127.5 62.08) (width 0.25) (layer "F.Cu") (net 2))
 (segment (start 123.15 62.5) (end 127.08 62.5) (width 0.25) (layer "F.Cu") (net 2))
 (segment (start 123.15 64.35) (end 123 64.5) (width 0.25) (layer "F.Cu") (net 2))
 (segment (start 123.15 62.5) (end 123.15 64.35) (width 0.25) (layer "F.Cu") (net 2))
 (segment (start 119 62.5) (end 116.225 62.5) (width 0.25) (layer "F.Cu") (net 1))
 (segment (start 119 62.5) (end 121.5 62.5) (width 0.25) (layer "F.Cu") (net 1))
 (segment (start 118 63.15) (end 116.225 63.15) (width 0.25) (layer "F.Cu") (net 10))
 (segment (start 119 64.15) (end 118 63.15) (width 0.25) (layer "F.Cu") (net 10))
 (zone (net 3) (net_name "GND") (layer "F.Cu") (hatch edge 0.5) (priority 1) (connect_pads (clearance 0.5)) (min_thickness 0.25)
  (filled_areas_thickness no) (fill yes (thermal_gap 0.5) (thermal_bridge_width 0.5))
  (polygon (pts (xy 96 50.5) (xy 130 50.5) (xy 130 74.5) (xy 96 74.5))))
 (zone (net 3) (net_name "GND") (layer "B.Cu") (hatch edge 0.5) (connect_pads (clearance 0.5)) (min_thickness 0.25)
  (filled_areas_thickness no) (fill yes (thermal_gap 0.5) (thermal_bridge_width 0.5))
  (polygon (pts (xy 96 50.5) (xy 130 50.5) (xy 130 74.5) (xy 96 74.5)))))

